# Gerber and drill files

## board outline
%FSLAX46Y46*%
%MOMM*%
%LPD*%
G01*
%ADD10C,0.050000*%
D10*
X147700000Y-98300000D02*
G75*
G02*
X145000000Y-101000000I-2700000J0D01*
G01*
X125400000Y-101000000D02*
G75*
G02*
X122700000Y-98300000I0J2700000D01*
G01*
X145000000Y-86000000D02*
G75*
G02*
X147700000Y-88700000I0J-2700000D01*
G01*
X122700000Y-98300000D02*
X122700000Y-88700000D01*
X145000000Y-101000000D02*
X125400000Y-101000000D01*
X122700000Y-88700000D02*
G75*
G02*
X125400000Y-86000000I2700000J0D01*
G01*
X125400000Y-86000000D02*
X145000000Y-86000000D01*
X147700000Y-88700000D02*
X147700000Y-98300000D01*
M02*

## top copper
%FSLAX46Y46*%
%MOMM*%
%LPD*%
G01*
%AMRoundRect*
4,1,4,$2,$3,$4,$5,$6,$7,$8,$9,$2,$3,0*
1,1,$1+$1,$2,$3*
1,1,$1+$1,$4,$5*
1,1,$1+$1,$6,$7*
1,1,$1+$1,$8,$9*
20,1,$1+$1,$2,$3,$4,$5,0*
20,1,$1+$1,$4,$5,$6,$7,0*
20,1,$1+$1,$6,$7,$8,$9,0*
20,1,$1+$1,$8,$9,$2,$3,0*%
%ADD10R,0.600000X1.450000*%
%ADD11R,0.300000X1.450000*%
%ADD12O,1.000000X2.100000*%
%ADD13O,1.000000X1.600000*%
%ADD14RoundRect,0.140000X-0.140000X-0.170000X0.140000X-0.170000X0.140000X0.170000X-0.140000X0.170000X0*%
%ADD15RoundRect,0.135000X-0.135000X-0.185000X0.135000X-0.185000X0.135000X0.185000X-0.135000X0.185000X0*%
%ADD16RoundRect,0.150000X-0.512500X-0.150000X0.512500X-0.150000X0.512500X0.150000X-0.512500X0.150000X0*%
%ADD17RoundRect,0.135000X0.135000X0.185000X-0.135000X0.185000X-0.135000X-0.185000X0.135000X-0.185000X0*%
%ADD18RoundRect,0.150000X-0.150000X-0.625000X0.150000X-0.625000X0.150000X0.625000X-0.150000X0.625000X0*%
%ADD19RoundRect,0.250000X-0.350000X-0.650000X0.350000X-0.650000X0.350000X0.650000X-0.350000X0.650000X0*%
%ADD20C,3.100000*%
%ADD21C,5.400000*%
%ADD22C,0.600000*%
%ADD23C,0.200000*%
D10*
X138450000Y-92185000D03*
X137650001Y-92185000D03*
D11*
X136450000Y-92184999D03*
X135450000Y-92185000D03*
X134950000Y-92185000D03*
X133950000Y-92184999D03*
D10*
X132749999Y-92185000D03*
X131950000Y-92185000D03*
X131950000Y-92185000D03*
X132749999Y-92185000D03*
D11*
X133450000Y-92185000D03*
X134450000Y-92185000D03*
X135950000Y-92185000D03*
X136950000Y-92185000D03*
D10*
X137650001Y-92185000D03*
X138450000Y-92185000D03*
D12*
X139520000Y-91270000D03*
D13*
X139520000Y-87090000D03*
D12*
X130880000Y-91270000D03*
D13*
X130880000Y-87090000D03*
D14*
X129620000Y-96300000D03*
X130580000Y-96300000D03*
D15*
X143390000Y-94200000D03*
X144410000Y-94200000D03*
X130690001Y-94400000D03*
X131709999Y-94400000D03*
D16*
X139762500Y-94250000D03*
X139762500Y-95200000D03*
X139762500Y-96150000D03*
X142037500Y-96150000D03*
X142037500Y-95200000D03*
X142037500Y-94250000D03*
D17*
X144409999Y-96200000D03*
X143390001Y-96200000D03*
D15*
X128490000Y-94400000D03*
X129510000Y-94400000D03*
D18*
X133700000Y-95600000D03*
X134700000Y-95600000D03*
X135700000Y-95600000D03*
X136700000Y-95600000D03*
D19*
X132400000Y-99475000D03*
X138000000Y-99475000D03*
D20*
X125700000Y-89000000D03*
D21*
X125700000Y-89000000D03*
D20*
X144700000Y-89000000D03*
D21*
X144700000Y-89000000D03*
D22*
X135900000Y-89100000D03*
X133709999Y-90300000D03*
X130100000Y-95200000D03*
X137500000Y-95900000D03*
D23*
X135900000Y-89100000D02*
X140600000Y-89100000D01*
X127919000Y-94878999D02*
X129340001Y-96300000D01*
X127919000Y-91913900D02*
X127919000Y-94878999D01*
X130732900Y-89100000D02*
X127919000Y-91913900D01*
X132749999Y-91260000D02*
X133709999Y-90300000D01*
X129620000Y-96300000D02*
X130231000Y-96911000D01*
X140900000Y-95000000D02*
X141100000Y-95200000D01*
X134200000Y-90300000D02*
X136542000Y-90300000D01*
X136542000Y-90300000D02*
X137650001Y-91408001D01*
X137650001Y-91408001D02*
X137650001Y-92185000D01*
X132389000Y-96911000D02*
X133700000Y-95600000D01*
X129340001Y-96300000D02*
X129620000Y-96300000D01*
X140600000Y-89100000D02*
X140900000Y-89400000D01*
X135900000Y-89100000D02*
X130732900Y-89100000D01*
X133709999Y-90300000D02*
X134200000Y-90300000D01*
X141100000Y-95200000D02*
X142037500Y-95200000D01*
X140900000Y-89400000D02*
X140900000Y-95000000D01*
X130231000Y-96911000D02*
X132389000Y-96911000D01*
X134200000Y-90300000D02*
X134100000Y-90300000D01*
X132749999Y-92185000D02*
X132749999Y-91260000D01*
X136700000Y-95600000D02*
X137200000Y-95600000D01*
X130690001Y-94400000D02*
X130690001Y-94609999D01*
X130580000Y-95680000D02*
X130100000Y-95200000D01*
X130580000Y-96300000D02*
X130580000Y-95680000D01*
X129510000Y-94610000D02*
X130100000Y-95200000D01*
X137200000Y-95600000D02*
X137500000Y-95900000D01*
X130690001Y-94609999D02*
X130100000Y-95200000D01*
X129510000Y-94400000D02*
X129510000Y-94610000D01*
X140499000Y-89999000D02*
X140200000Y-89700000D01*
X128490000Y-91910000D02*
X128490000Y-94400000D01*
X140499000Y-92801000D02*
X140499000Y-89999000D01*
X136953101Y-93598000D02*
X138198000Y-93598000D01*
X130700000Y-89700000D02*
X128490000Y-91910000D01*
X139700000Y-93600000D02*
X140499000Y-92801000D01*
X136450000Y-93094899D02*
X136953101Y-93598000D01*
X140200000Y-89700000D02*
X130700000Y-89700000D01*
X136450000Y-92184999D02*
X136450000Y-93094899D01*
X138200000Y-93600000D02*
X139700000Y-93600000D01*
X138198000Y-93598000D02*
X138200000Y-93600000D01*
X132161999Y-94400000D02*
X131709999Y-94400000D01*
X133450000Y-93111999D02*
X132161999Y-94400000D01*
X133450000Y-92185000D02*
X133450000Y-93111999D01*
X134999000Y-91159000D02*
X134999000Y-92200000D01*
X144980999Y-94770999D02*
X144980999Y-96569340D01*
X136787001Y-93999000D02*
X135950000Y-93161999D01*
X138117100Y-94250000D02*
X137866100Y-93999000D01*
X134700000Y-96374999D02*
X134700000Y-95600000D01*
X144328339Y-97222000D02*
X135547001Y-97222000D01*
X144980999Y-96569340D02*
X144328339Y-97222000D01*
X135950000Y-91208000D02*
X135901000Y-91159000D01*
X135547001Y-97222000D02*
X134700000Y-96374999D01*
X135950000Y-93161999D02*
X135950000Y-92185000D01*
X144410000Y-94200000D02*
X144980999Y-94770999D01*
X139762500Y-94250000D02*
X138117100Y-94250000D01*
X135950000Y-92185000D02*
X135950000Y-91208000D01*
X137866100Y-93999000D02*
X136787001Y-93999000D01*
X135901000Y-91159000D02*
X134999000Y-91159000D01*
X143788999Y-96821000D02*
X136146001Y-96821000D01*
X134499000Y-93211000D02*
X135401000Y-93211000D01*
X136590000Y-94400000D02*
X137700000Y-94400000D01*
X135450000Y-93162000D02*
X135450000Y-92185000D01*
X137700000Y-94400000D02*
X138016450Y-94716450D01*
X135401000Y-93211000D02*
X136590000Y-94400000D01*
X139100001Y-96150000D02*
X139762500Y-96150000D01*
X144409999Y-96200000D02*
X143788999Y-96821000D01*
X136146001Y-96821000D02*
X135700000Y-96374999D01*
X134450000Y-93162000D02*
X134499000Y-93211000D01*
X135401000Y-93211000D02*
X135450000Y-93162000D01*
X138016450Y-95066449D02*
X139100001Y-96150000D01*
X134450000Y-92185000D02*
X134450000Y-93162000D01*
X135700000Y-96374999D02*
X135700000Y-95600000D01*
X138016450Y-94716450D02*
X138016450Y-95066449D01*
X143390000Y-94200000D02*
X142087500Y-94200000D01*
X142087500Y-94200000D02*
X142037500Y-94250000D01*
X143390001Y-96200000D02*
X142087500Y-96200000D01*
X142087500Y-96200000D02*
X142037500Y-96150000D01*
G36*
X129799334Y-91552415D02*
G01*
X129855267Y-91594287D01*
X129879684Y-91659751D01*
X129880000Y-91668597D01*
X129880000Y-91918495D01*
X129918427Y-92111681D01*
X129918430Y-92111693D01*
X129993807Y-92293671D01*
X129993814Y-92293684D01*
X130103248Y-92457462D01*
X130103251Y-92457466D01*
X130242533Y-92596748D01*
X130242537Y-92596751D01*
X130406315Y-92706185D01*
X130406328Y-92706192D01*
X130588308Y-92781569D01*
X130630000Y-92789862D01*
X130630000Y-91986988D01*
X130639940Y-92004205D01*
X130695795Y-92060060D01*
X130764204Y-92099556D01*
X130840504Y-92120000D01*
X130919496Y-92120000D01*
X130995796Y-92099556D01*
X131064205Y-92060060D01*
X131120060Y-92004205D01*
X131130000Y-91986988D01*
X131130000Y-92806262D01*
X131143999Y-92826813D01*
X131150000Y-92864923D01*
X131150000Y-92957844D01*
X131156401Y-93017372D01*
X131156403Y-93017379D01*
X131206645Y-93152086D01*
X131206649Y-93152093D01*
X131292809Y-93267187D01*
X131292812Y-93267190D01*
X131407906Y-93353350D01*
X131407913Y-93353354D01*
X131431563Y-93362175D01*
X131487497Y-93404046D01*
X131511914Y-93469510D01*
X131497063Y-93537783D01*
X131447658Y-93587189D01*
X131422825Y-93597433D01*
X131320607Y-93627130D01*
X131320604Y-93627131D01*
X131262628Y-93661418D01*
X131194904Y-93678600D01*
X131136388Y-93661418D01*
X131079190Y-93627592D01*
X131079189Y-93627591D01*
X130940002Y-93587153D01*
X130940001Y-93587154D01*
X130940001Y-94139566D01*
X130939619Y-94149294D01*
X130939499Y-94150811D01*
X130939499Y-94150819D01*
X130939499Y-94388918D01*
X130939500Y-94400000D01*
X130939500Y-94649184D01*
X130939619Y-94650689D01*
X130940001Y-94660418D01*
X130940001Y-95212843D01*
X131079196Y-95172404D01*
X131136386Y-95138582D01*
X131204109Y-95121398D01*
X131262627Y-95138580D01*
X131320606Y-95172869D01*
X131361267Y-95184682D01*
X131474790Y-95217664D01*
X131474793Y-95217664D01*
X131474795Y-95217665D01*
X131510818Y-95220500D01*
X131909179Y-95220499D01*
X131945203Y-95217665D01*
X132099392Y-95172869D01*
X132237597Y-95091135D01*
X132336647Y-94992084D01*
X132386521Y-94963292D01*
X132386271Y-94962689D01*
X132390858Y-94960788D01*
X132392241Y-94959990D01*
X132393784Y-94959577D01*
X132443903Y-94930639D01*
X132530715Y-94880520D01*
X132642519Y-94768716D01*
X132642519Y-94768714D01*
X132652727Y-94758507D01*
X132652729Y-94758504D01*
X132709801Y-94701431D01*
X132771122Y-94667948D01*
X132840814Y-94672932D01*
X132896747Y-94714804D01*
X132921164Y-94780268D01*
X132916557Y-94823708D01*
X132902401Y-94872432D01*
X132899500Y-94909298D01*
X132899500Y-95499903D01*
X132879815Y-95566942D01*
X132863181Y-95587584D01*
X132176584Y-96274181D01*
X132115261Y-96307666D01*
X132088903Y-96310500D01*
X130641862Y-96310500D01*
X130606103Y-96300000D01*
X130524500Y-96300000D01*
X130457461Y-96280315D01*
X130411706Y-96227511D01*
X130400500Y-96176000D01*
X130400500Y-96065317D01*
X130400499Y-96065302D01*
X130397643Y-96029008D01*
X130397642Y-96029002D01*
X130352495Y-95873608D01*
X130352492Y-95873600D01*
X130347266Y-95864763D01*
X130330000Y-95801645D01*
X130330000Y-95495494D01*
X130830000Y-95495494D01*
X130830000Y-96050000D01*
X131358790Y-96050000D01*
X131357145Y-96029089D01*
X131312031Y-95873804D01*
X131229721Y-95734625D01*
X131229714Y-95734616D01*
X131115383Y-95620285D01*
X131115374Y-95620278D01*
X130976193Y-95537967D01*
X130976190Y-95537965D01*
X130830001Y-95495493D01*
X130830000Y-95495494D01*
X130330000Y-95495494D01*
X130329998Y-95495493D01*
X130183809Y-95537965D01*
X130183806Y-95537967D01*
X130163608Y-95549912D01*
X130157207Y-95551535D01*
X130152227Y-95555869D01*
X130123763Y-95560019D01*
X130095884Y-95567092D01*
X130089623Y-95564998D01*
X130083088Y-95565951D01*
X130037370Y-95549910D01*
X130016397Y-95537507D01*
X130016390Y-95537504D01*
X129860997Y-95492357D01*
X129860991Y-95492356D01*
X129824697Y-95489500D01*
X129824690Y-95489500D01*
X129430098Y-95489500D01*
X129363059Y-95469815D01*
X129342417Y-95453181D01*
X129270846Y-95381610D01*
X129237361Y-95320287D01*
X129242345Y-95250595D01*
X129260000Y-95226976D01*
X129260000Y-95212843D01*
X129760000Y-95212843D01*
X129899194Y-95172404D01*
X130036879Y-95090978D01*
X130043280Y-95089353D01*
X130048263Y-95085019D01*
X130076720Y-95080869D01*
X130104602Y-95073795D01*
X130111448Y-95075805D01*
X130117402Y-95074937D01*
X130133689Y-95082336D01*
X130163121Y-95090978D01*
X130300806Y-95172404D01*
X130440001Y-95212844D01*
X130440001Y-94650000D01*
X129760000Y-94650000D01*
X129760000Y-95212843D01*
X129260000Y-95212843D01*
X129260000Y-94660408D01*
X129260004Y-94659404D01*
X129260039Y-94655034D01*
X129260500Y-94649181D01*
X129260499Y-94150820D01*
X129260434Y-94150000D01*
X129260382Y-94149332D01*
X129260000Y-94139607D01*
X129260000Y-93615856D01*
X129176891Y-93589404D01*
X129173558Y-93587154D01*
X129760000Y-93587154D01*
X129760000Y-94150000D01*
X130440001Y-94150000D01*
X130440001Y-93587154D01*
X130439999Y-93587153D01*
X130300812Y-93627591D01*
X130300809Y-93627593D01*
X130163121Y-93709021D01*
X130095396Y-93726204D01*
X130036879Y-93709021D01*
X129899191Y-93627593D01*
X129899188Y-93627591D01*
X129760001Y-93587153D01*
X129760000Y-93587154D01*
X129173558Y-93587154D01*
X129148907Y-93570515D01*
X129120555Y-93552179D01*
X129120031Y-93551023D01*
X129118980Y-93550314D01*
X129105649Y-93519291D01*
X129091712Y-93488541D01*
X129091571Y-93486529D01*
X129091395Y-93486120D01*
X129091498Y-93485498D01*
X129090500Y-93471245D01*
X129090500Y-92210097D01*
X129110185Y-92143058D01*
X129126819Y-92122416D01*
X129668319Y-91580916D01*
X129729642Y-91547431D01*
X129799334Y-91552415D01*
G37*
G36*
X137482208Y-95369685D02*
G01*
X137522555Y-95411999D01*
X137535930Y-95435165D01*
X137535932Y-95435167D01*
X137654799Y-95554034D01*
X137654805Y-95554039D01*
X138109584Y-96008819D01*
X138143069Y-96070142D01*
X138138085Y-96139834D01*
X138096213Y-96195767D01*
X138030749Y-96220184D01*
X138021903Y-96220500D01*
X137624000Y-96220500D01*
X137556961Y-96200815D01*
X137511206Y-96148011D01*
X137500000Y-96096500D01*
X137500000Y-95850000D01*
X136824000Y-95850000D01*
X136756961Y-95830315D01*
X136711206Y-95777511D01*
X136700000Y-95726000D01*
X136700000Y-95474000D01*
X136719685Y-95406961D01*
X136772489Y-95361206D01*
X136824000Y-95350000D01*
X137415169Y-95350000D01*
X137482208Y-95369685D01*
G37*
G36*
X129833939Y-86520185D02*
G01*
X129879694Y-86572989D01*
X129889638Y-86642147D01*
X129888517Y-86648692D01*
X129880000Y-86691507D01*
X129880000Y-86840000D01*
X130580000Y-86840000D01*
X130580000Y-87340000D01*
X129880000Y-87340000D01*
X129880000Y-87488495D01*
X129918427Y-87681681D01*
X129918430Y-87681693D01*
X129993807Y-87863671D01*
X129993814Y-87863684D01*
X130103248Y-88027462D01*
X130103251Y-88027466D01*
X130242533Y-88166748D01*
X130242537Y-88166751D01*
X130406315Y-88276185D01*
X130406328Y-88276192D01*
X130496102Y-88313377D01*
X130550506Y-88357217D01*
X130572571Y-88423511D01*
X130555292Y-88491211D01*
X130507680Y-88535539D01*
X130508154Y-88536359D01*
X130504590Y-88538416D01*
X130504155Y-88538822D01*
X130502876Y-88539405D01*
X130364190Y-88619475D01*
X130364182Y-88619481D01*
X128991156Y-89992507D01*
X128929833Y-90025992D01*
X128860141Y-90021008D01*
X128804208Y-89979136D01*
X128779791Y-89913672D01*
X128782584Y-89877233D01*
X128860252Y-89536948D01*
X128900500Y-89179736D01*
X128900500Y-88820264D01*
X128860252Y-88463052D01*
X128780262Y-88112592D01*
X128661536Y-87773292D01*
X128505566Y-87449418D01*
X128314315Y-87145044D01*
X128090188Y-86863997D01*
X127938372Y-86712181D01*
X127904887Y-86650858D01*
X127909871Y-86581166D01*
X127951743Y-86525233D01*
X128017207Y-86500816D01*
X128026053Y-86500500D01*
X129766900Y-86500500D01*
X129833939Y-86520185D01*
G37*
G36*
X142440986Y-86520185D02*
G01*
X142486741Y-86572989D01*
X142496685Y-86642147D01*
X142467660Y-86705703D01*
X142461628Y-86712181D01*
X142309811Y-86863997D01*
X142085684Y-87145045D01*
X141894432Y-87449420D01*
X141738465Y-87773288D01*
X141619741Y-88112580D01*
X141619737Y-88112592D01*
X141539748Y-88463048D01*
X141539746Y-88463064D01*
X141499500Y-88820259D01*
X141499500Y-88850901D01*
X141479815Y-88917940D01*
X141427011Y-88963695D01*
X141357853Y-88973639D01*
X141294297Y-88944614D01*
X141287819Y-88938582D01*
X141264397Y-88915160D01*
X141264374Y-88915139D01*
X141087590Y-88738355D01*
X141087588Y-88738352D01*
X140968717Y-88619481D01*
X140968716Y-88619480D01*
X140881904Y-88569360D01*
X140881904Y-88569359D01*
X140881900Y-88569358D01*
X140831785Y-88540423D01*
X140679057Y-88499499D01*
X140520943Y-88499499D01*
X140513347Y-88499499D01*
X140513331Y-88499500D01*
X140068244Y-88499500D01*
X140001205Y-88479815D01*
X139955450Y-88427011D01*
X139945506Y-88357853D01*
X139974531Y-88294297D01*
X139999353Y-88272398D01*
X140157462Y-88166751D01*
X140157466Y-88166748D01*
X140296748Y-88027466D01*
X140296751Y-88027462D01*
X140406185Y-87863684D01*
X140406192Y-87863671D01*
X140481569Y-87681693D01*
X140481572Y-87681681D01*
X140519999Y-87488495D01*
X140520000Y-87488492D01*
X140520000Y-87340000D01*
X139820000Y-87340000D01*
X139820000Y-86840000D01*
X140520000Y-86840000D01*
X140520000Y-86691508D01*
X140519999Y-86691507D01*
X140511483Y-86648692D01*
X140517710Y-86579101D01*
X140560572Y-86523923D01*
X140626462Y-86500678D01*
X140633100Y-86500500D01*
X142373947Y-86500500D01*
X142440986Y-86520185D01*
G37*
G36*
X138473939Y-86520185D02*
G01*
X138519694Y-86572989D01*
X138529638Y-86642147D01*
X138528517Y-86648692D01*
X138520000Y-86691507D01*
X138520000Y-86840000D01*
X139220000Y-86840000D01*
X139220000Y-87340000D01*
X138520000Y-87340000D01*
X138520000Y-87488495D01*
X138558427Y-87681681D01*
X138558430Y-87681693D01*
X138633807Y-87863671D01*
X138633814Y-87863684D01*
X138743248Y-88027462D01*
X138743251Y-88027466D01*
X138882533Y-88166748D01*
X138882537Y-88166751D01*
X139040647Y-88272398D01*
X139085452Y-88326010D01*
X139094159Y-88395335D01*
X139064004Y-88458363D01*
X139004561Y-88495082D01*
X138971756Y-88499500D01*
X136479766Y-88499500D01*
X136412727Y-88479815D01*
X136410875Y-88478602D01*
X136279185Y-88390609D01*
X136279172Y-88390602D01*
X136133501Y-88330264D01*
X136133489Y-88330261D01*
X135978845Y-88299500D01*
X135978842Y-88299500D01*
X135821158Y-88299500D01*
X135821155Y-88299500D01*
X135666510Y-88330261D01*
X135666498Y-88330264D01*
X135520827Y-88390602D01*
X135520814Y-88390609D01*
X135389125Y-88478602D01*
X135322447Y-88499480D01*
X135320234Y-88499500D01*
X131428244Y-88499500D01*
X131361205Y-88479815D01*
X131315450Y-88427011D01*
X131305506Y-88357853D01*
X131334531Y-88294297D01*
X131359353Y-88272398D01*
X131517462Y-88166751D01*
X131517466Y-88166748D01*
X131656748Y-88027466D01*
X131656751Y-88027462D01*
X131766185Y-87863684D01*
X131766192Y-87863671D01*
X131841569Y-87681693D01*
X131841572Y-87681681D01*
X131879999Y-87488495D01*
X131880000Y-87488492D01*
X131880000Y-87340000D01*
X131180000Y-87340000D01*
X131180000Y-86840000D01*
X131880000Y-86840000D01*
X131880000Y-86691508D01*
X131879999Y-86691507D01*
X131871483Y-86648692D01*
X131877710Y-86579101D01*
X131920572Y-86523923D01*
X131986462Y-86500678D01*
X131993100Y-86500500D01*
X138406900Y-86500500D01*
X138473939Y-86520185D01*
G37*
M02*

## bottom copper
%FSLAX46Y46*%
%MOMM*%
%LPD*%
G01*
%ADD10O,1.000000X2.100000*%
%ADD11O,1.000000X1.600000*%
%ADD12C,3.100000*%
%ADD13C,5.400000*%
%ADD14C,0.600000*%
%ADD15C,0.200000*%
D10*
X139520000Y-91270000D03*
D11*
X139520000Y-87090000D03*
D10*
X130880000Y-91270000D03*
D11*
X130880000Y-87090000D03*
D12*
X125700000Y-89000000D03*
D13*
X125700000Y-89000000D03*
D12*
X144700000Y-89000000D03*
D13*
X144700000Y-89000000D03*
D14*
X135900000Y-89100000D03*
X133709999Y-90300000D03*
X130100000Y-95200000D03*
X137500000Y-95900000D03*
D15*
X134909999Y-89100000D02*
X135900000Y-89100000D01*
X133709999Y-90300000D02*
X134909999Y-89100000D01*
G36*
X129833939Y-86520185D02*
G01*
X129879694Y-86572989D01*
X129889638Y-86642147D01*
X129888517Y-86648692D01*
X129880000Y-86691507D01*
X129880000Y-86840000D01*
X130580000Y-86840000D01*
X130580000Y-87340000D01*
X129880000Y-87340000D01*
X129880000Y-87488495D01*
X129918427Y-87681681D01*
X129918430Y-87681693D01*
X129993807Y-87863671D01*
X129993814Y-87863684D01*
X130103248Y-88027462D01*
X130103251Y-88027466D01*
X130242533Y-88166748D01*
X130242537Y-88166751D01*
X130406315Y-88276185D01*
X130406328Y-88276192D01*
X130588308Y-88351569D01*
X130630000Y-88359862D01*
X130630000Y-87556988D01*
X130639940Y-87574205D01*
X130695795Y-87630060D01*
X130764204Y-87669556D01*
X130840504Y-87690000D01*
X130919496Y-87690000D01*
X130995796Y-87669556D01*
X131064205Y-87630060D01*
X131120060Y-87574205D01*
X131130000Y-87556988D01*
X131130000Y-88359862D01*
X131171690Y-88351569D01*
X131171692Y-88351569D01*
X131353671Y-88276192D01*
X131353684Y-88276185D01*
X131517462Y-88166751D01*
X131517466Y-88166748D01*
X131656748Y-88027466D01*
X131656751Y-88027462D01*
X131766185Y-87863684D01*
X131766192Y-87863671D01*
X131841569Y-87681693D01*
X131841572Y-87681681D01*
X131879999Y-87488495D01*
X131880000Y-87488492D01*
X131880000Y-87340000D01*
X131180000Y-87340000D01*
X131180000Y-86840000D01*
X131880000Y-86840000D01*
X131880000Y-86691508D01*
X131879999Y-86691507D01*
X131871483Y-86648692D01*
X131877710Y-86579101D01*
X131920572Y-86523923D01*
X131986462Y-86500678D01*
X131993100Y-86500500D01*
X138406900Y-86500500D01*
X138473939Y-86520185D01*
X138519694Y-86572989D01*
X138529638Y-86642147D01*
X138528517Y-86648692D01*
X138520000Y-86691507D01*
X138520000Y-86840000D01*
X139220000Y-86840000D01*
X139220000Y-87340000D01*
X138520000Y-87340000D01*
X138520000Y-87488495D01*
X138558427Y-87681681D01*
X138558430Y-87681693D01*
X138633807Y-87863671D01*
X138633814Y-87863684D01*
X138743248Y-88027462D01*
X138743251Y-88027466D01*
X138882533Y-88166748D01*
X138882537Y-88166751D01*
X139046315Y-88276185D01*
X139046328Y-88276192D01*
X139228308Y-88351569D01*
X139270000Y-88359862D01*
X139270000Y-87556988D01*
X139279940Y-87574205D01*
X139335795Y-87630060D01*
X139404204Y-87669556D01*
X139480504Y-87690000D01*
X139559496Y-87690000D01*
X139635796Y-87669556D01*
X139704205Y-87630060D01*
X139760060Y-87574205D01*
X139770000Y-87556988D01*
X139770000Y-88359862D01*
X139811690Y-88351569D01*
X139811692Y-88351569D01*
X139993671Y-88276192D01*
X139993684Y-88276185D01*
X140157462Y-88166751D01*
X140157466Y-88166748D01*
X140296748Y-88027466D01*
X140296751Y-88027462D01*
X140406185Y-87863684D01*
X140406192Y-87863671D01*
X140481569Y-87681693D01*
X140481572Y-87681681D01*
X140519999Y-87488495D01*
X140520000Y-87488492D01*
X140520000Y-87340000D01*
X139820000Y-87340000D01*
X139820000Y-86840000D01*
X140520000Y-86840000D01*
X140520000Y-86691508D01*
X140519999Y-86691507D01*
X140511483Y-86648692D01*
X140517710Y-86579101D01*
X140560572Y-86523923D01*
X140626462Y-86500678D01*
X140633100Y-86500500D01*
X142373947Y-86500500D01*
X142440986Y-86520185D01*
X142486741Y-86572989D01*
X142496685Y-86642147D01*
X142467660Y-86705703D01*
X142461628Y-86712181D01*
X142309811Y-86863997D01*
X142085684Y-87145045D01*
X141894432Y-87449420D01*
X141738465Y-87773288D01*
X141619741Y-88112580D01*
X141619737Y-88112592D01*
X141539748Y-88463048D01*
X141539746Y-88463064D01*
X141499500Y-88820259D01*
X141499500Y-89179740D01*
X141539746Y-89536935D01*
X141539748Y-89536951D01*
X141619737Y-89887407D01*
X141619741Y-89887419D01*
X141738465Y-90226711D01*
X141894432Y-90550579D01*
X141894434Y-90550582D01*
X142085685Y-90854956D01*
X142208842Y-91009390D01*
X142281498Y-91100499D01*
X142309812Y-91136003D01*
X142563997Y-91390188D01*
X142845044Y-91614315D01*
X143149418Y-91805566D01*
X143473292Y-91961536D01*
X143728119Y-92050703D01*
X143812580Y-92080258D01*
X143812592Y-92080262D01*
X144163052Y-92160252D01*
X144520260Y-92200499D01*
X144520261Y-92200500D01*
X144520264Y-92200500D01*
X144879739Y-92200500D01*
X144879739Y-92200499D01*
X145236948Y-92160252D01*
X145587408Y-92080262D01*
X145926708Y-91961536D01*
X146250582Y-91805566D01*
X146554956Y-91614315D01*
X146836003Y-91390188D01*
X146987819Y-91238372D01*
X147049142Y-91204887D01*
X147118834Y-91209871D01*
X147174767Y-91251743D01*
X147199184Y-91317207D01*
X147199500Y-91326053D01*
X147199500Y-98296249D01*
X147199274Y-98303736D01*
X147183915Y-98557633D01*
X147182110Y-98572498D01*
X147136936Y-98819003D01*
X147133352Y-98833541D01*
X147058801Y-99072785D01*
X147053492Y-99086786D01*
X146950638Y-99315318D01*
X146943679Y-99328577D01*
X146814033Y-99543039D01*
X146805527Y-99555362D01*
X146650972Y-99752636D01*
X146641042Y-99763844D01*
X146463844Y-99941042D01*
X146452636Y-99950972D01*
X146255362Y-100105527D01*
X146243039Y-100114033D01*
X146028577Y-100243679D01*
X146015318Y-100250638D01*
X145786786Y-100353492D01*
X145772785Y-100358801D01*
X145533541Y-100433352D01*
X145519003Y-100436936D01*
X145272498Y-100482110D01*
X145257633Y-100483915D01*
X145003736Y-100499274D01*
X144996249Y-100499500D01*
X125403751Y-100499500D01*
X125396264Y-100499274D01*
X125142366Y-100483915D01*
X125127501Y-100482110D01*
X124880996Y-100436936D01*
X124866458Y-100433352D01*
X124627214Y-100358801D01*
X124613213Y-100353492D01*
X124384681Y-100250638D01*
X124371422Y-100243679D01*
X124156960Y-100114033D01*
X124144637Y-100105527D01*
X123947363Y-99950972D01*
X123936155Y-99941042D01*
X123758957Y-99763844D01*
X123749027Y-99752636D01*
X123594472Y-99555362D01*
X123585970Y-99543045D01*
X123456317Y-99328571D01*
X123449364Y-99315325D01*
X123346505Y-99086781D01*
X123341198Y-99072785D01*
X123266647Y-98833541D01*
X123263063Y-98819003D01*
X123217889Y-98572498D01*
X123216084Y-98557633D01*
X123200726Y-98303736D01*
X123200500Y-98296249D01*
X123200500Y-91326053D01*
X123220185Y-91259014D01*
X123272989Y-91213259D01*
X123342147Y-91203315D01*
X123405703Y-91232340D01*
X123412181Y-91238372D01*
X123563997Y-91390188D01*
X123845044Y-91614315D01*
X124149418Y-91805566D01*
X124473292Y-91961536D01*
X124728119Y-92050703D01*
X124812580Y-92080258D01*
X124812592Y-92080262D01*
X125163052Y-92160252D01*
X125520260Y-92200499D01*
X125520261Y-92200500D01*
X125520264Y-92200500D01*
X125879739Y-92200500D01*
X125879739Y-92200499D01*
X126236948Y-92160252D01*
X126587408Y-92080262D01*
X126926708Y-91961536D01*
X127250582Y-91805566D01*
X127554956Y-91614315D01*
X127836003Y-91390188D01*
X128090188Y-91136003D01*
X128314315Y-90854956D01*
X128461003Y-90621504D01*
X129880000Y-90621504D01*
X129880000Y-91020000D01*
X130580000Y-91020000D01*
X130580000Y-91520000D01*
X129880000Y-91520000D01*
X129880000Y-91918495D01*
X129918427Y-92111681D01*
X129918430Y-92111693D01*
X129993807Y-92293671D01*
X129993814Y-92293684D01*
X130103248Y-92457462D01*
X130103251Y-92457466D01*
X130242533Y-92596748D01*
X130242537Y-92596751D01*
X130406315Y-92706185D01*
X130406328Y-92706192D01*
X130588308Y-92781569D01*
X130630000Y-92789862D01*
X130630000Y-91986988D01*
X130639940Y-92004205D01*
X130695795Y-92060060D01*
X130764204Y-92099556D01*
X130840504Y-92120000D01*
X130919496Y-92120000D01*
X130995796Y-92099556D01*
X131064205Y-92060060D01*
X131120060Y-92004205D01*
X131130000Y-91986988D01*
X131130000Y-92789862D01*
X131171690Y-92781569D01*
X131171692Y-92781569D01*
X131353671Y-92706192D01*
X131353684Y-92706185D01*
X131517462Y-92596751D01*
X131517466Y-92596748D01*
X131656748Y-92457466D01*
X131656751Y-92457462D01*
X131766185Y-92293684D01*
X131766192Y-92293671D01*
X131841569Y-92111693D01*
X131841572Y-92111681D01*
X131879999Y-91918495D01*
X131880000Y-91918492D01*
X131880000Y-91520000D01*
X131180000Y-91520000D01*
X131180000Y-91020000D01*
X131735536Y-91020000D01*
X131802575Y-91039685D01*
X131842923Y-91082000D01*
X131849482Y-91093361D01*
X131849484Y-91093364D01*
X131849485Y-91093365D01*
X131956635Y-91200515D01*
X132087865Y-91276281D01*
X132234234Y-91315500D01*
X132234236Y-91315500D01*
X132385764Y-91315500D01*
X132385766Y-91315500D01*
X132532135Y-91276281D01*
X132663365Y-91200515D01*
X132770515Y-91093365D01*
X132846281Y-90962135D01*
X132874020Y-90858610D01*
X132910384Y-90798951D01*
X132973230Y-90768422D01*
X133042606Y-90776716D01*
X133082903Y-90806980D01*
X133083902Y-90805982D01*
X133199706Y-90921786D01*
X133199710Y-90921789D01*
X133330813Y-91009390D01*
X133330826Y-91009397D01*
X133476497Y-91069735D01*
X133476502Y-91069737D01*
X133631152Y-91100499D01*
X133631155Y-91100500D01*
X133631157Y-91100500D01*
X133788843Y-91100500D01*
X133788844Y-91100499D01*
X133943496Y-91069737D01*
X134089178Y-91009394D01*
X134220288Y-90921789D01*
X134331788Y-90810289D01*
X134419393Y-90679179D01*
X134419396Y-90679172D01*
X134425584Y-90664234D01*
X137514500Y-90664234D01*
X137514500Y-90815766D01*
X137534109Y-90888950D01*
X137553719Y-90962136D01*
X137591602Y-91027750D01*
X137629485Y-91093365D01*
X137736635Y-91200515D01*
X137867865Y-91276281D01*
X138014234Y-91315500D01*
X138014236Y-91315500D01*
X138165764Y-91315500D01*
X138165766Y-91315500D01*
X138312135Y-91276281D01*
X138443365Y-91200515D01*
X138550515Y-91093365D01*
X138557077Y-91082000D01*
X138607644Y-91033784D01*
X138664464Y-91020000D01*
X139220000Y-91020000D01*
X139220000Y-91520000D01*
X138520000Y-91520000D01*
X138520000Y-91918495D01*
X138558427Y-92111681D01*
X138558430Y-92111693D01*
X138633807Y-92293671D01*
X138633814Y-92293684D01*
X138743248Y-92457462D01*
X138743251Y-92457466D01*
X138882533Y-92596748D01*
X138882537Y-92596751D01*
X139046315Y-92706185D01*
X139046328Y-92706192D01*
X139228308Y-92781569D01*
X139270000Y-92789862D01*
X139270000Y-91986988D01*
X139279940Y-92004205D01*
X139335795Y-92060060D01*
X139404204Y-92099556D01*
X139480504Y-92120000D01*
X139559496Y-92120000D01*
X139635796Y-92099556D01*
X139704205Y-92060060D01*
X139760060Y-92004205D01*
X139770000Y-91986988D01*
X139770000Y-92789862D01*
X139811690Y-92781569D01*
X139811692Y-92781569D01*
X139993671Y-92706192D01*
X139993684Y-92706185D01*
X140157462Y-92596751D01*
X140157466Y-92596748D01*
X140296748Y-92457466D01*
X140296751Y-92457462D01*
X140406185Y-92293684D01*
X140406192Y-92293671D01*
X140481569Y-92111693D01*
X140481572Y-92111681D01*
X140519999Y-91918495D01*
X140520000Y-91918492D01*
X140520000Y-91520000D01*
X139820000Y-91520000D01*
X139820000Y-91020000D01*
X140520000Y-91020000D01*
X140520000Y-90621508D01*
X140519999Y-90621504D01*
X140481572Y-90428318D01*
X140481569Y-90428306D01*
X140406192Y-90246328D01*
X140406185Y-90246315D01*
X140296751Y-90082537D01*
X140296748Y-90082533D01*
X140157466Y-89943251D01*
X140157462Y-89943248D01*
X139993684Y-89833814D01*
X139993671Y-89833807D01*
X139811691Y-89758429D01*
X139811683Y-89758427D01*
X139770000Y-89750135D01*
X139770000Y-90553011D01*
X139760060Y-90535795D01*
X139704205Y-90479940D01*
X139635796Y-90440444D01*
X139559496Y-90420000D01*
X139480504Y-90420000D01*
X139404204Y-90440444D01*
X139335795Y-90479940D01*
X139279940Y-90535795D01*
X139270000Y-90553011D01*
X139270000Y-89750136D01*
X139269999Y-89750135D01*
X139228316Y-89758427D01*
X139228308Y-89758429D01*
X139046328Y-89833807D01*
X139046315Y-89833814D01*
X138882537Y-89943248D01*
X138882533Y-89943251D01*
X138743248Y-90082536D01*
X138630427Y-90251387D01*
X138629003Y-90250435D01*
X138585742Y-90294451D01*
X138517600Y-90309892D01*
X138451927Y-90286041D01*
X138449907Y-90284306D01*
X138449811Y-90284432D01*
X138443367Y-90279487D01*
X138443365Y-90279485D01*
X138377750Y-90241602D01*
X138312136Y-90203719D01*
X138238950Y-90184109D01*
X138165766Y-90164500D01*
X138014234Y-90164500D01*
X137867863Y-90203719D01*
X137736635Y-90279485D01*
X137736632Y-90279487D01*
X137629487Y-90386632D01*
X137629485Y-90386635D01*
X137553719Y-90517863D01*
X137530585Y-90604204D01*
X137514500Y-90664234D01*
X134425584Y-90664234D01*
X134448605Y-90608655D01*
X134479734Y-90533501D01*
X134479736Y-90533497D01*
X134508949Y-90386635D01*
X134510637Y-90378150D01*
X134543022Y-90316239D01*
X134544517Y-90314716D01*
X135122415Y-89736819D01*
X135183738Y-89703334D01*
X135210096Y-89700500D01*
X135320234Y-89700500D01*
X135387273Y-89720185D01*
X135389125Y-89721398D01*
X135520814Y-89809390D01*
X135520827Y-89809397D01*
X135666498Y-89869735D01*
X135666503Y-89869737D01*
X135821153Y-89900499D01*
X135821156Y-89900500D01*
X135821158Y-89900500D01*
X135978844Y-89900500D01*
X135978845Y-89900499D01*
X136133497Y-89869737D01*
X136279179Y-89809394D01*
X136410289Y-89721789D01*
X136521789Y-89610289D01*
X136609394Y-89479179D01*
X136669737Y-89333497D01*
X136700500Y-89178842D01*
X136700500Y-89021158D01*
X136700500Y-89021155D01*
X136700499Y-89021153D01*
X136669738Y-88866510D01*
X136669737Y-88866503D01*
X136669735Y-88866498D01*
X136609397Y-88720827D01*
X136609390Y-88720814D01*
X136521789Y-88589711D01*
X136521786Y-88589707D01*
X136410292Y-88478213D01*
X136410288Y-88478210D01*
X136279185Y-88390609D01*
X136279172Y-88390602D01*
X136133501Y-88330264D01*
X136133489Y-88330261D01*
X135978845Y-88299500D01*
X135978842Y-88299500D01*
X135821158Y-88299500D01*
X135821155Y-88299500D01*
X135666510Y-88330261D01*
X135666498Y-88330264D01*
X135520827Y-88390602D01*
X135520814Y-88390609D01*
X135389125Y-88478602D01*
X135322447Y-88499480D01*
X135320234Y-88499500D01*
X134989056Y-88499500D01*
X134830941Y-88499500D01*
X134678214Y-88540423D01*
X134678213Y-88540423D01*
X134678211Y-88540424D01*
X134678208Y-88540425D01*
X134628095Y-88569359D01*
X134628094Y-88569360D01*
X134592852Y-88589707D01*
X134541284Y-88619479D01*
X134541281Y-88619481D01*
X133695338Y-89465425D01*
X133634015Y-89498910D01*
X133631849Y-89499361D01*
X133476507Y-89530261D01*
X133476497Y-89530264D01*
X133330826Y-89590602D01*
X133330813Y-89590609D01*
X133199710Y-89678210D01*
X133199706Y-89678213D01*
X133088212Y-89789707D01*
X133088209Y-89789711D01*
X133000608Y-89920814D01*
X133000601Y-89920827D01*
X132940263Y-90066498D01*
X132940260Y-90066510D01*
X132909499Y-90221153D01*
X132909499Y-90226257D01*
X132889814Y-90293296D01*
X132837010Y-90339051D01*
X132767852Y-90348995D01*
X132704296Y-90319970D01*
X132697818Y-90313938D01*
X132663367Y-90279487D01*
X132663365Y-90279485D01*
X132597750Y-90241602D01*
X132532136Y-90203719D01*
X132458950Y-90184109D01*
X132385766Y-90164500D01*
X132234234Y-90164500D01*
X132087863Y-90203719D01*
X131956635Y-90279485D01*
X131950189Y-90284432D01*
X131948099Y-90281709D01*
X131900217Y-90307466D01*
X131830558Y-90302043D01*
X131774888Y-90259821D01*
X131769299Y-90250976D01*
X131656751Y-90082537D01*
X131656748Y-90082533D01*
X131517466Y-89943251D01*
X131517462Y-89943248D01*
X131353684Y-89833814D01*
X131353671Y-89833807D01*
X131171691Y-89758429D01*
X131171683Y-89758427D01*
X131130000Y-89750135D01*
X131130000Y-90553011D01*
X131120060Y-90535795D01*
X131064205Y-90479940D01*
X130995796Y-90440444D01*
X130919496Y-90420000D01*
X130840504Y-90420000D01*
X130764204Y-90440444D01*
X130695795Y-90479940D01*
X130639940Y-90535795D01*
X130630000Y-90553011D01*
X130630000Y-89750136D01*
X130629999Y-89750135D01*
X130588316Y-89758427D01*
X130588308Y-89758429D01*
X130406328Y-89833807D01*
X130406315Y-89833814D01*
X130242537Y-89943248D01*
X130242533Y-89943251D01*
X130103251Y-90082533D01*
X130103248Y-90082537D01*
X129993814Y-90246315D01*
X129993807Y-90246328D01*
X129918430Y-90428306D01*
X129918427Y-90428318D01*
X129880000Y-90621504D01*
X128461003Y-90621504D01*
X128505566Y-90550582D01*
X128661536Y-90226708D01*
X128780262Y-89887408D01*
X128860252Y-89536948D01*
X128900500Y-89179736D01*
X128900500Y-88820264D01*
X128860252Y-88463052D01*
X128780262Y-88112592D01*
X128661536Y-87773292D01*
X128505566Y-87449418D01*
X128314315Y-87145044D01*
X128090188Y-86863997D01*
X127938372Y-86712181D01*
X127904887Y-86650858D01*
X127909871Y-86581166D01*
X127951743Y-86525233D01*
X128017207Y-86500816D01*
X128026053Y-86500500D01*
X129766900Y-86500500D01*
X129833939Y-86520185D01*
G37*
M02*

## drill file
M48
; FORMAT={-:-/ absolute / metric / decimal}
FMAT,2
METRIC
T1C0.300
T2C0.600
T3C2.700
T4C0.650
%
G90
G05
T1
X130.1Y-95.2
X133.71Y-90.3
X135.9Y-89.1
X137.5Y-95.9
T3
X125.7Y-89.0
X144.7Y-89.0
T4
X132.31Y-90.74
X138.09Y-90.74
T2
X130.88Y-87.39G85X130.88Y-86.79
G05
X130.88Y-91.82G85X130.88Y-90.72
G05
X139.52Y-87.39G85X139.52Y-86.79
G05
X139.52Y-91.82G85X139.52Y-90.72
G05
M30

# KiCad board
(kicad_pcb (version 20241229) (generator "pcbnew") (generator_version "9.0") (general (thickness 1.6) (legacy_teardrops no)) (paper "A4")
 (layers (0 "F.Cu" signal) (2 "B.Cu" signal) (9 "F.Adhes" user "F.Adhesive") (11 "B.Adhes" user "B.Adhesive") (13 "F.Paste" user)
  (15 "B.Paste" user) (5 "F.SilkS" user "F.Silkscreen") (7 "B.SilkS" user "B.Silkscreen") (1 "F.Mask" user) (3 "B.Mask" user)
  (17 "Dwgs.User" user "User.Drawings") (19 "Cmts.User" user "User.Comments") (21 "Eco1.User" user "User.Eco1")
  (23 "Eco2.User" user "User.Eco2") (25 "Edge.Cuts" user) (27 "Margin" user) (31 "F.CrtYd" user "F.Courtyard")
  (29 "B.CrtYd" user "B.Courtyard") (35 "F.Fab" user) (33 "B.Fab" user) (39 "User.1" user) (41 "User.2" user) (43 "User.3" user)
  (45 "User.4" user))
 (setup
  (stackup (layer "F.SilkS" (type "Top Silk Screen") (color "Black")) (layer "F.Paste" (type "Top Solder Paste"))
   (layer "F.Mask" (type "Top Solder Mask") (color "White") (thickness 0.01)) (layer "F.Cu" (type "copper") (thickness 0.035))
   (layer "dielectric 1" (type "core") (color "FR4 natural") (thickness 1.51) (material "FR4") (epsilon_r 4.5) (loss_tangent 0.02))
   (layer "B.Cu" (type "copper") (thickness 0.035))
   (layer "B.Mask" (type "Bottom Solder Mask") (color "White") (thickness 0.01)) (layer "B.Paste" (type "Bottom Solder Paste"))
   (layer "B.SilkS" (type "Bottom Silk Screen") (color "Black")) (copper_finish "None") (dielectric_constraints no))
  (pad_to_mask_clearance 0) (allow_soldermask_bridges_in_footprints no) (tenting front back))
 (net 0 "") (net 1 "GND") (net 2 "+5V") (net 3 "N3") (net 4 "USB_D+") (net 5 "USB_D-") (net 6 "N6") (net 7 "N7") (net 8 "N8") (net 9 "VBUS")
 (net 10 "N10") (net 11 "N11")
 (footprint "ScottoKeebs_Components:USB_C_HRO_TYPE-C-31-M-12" (layer "F.Cu") (at 135.2 88.14 180)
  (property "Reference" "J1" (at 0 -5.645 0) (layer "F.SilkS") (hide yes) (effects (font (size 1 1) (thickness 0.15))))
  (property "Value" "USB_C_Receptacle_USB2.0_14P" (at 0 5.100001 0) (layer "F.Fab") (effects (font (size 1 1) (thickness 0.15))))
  (pad "" np_thru_hole circle (at -2.89 -2.6 180) (size 0.65 0.65) (drill 0.65) (layers "*.Cu" "*.Mask"))
  (pad "" np_thru_hole circle (at 2.89 -2.6 180) (size 0.65 0.65) (drill 0.65) (layers "*.Cu" "*.Mask"))
  (pad "A1" smd rect (at -3.25 -4.045 180) (size 0.6 1.45) (layers "F.Cu" "F.Mask" "F.Paste") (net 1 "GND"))
  (pad "A4" smd rect (at -2.450001 -4.045 180) (size 0.6 1.45) (layers "F.Cu" "F.Mask" "F.Paste") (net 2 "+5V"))
  (pad "A5" smd rect (at -1.25 -4.044999 180) (size 0.3 1.45) (layers "F.Cu" "F.Mask" "F.Paste") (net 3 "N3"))
  (pad "A6" smd rect (at -0.25 -4.045 180) (size 0.3 1.45) (layers "F.Cu" "F.Mask" "F.Paste") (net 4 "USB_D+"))
  (pad "A7" smd rect (at 0.25 -4.045 180) (size 0.3 1.45) (layers "F.Cu" "F.Mask" "F.Paste") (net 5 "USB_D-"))
  (pad "A8" smd rect (at 1.25 -4.044999 180) (size 0.3 1.45) (layers "F.Cu" "F.Mask" "F.Paste"))
  (pad "A9" smd rect (at 2.450001 -4.045 180) (size 0.6 1.45) (layers "F.Cu" "F.Mask" "F.Paste") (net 2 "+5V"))
  (pad "A12" smd rect (at 3.25 -4.045 180) (size 0.6 1.45) (layers "F.Cu" "F.Mask" "F.Paste") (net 1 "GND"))
  (pad "B1" smd rect (at 3.25 -4.045 180) (size 0.6 1.45) (layers "F.Cu" "F.Mask" "F.Paste") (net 1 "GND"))
  (pad "B4" smd rect (at 2.450001 -4.045 180) (size 0.6 1.45) (layers "F.Cu" "F.Mask" "F.Paste") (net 2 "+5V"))
  (pad "B5" smd rect (at 1.75 -4.045 180) (size 0.3 1.45) (layers "F.Cu" "F.Mask" "F.Paste") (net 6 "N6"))
  (pad "B6" smd rect (at 0.75 -4.045 180) (size 0.3 1.45) (layers "F.Cu" "F.Mask" "F.Paste") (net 4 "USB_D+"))
  (pad "B7" smd rect (at -0.75 -4.045 180) (size 0.3 1.45) (layers "F.Cu" "F.Mask" "F.Paste") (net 5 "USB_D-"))
  (pad "B8" smd rect (at -1.75 -4.045 180) (size 0.3 1.45) (layers "F.Cu" "F.Mask" "F.Paste"))
  (pad "B9" smd rect (at -2.450001 -4.045 180) (size 0.6 1.45) (layers "F.Cu" "F.Mask" "F.Paste") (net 2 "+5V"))
  (pad "B12" smd rect (at -3.25 -4.045 180) (size 0.6 1.45) (layers "F.Cu" "F.Mask" "F.Paste") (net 1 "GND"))
  (pad "S1" thru_hole oval (at -4.32 -3.13 180) (size 1 2.1) (drill oval 0.6 1.7) (layers "*.Cu" "*.Mask") (remove_unused_layers no)
   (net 1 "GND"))
  (pad "S1" thru_hole oval (at -4.32 1.05 180) (size 1 1.6) (drill oval 0.6 1.2) (layers "*.Cu" "*.Mask") (remove_unused_layers no)
   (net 1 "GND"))
  (pad "S1" thru_hole oval (at 4.32 -3.13 180) (size 1 2.1) (drill oval 0.6 1.7) (layers "*.Cu" "*.Mask") (remove_unused_layers no)
   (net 1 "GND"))
  (pad "S1" thru_hole oval (at 4.32 1.05 180) (size 1 1.6) (drill oval 0.6 1.2) (layers "*.Cu" "*.Mask") (remove_unused_layers no)
   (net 1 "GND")))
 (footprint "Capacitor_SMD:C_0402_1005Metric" (layer "F.Cu") (at 130.1 96.3)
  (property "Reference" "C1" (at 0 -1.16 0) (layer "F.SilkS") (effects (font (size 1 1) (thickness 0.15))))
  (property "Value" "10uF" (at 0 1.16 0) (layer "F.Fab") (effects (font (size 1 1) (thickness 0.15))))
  (pad "1" smd roundrect (at -0.48 0) (size 0.56 0.62) (layers "F.Cu" "F.Mask" "F.Paste") (roundrect_rratio 0.25) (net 2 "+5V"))
  (pad "2" smd roundrect (at 0.48 0) (size 0.56 0.62) (layers "F.Cu" "F.Mask" "F.Paste") (roundrect_rratio 0.25) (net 1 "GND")))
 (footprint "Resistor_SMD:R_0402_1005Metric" (layer "F.Cu") (at 143.9 94.2)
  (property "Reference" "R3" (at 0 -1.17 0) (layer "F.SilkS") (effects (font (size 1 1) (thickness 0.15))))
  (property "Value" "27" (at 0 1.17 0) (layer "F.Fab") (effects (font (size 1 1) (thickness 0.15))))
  (pad "1" smd roundrect (at -0.51 0) (size 0.54 0.64) (layers "F.Cu" "F.Mask" "F.Paste") (roundrect_rratio 0.25) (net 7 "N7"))
  (pad "2" smd roundrect (at 0.51 0) (size 0.54 0.64) (layers "F.Cu" "F.Mask" "F.Paste") (roundrect_rratio 0.25) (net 4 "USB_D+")))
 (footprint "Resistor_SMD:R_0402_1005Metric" (layer "F.Cu") (at 131.2 94.4)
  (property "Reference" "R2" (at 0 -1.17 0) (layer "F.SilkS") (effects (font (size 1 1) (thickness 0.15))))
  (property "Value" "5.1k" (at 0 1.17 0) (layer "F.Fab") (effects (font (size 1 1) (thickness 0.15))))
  (pad "1" smd roundrect (at -0.509999 0) (size 0.54 0.64) (layers "F.Cu" "F.Mask" "F.Paste") (roundrect_rratio 0.25) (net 1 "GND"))
  (pad "2" smd roundrect (at 0.509999 0) (size 0.54 0.64) (layers "F.Cu" "F.Mask" "F.Paste") (roundrect_rratio 0.25) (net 6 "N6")))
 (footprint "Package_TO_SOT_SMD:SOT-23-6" (layer "F.Cu") (at 140.9 95.2)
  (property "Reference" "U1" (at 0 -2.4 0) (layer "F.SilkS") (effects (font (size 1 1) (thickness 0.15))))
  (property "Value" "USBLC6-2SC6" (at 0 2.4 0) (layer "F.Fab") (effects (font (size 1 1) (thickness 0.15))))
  (pad "1" smd roundrect (at -1.1375 -0.95) (size 1.325 0.6) (layers "F.Cu" "F.Mask" "F.Paste") (roundrect_rratio 0.25) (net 4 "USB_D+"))
  (pad "2" smd roundrect (at -1.1375 0) (size 1.325 0.6) (layers "F.Cu" "F.Mask" "F.Paste") (roundrect_rratio 0.25) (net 1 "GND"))
  (pad "3" smd roundrect (at -1.1375 0.95) (size 1.325 0.6) (layers "F.Cu" "F.Mask" "F.Paste") (roundrect_rratio 0.25) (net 5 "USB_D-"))
  (pad "4" smd roundrect (at 1.1375 0.95) (size 1.325 0.6) (layers "F.Cu" "F.Mask" "F.Paste") (roundrect_rratio 0.25) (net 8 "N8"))
  (pad "5" smd roundrect (at 1.1375 0) (size 1.325 0.6) (layers "F.Cu" "F.Mask" "F.Paste") (roundrect_rratio 0.25) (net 2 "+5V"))
  (pad "6" smd roundrect (at 1.1375 -0.95) (size 1.325 0.6) (layers "F.Cu" "F.Mask" "F.Paste") (roundrect_rratio 0.25) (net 7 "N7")))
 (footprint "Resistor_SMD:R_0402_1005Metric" (layer "F.Cu") (at 143.9 96.2 180)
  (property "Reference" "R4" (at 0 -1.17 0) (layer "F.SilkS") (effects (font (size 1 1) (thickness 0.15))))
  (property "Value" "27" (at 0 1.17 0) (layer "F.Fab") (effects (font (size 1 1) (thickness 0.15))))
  (pad "1" smd roundrect (at -0.509999 0 180) (size 0.54 0.64) (layers "F.Cu" "F.Mask" "F.Paste") (roundrect_rratio 0.25) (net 5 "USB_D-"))
  (pad "2" smd roundrect (at 0.509999 0 180) (size 0.54 0.64) (layers "F.Cu" "F.Mask" "F.Paste") (roundrect_rratio 0.25) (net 8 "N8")))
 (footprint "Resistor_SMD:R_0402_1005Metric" (layer "F.Cu") (at 129 94.4)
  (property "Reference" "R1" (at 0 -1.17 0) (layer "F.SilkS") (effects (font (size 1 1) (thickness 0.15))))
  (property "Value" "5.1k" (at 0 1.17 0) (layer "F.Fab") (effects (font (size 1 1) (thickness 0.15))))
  (pad "1" smd roundrect (at -0.51 0) (size 0.54 0.64) (layers "F.Cu" "F.Mask" "F.Paste") (roundrect_rratio 0.25) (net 3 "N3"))
  (pad "2" smd roundrect (at 0.51 0) (size 0.54 0.64) (layers "F.Cu" "F.Mask" "F.Paste") (roundrect_rratio 0.25) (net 1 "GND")))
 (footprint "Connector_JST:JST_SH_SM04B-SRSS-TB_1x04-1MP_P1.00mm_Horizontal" (layer "F.Cu") (at 135.2 97.6)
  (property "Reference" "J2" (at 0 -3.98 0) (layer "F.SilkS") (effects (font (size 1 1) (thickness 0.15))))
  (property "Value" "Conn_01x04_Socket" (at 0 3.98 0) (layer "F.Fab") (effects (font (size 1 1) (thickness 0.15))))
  (pad "1" smd roundrect (at -1.5 -2) (size 0.6 1.55) (layers "F.Cu" "F.Mask" "F.Paste") (roundrect_rratio 0.25) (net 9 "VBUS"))
  (pad "2" smd roundrect (at -0.5 -2) (size 0.6 1.55) (layers "F.Cu" "F.Mask" "F.Paste") (roundrect_rratio 0.25) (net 5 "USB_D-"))
  (pad "3" smd roundrect (at 0.5 -2) (size 0.6 1.55) (layers "F.Cu" "F.Mask" "F.Paste") (roundrect_rratio 0.25) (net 4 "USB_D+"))
  (pad "4" smd roundrect (at 1.5 -2) (size 0.6 1.55) (layers "F.Cu" "F.Mask" "F.Paste") (roundrect_rratio 0.25) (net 1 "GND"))
  (pad "MP" smd roundrect (at -2.8 1.875) (size 1.2 1.8) (layers "F.Cu" "F.Mask" "F.Paste") (roundrect_rratio 0.208333))
  (pad "MP" smd roundrect (at 2.8 1.875) (size 1.2 1.8) (layers "F.Cu" "F.Mask" "F.Paste") (roundrect_rratio 0.208333)))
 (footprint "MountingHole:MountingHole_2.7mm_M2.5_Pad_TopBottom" (layer "B.Cu") (at 125.7 89 180)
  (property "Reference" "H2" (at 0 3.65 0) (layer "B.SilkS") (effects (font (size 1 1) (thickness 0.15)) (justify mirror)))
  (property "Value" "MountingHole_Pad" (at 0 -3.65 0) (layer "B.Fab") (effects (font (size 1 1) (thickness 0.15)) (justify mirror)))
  (pad "1" thru_hole circle (at 0 0 180) (size 3.1 3.1) (drill 2.7) (layers "*.Cu" "*.Mask") (remove_unused_layers no) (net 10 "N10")
   (zone_connect 2))
  (pad "1" connect circle (at 0 0 180) (size 5.4 5.4) (layers "F.Cu" "F.Mask") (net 10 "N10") (zone_connect 2))
  (pad "1" connect circle (at 0 0 180) (size 5.4 5.4) (layers "B.Cu" "B.Mask") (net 10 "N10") (zone_connect 2)))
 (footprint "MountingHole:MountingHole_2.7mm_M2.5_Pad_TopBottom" (layer "B.Cu") (at 144.7 89 180)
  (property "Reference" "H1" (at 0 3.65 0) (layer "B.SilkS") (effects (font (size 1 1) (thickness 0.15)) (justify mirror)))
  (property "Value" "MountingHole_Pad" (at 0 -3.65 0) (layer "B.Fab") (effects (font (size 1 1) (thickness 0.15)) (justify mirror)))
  (pad "1" thru_hole circle (at 0 0 180) (size 3.1 3.1) (drill 2.7) (layers "*.Cu" "*.Mask") (remove_unused_layers no) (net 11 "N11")
   (zone_connect 2))
  (pad "1" connect circle (at 0 0 180) (size 5.4 5.4) (layers "F.Cu" "F.Mask") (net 11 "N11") (zone_connect 2))
  (pad "1" connect circle (at 0 0 180) (size 5.4 5.4) (layers "B.Cu" "B.Mask") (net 11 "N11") (zone_connect 2)))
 (gr_arc (start 147.7 98.3) (mid 146.909188 100.209188) (end 145 101) (stroke (width 0.05) (type default)) (layer "Edge.Cuts"))
 (gr_arc (start 125.4 101) (mid 123.490812 100.209188) (end 122.7 98.3) (stroke (width 0.05) (type default)) (layer "Edge.Cuts"))
 (gr_arc (start 145 86) (mid 146.909188 86.790812) (end 147.7 88.7) (stroke (width 0.05) (type default)) (layer "Edge.Cuts"))
 (gr_line (start 122.7 98.3) (end 122.7 88.7) (stroke (width 0.05) (type default)) (layer "Edge.Cuts"))
 (gr_line (start 145 101) (end 125.4 101) (stroke (width 0.05) (type default)) (layer "Edge.Cuts"))
 (gr_arc (start 122.7 88.7) (mid 123.490812 86.790812) (end 125.4 86) (stroke (width 0.05) (type default)) (layer "Edge.Cuts"))
 (gr_line (start 125.4 86) (end 145 86) (stroke (width 0.05) (type default)) (layer "Edge.Cuts"))
 (gr_line (start 147.7 88.7) (end 147.7 98.3) (stroke (width 0.05) (type default)) (layer "Edge.Cuts"))
 (segment (start 135.9 89.1) (end 140.6 89.1) (width 0.2) (layer "F.Cu") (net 2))
 (segment (start 127.919 94.878999) (end 129.340001 96.3) (width 0.2) (layer "F.Cu") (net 2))
 (segment (start 127.919 91.9139) (end 127.919 94.878999) (width 0.2) (layer "F.Cu") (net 2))
 (segment (start 130.7329 89.1) (end 127.919 91.9139) (width 0.2) (layer "F.Cu") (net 2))
 (segment (start 132.749999 91.26) (end 133.709999 90.3) (width 0.2) (layer "F.Cu") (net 2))
 (segment (start 129.62 96.3) (end 130.231 96.911) (width 0.2) (layer "F.Cu") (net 2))
 (segment (start 140.9 95) (end 141.1 95.2) (width 0.2) (layer "F.Cu") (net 2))
 (segment (start 134.2 90.3) (end 136.542 90.3) (width 0.2) (layer "F.Cu") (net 2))
 (segment (start 136.542 90.3) (end 137.650001 91.408001) (width 0.2) (layer "F.Cu") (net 2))
 (segment (start 137.650001 91.408001) (end 137.650001 92.185) (width 0.2) (layer "F.Cu") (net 2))
 (segment (start 132.389 96.911) (end 133.7 95.6) (width 0.2) (layer "F.Cu") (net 2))
 (segment (start 129.340001 96.3) (end 129.62 96.3) (width 0.2) (layer "F.Cu") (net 2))
 (segment (start 140.6 89.1) (end 140.9 89.4) (width 0.2) (layer "F.Cu") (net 2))
 (segment (start 135.9 89.1) (end 130.7329 89.1) (width 0.2) (layer "F.Cu") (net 2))
 (segment (start 133.709999 90.3) (end 134.2 90.3) (width 0.2) (layer "F.Cu") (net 2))
 (segment (start 141.1 95.2) (end 142.0375 95.2) (width 0.2) (layer "F.Cu") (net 2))
 (segment (start 140.9 89.4) (end 140.9 95) (width 0.2) (layer "F.Cu") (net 2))
 (segment (start 130.231 96.911) (end 132.389 96.911) (width 0.2) (layer "F.Cu") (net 2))
 (segment (start 134.2 90.3) (end 134.1 90.3) (width 0.2) (layer "F.Cu") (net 2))
 (segment (start 132.749999 92.185) (end 132.749999 91.26) (width 0.2) (layer "F.Cu") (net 2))
 (via (at 135.9 89.1) (size 0.6) (drill 0.3) (layers "F.Cu" "B.Cu") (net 2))
 (via (at 133.709999 90.3) (size 0.6) (drill 0.3) (layers "F.Cu" "B.Cu") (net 2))
 (segment (start 134.909999 89.1) (end 135.9 89.1) (width 0.2) (layer "B.Cu") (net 2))
 (segment (start 133.709999 90.3) (end 134.909999 89.1) (width 0.2) (layer "B.Cu") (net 2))
 (segment (start 136.7 95.6) (end 137.2 95.6) (width 0.2) (layer "F.Cu") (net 1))
 (segment (start 130.690001 94.4) (end 130.690001 94.609999) (width 0.2) (layer "F.Cu") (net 1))
 (segment (start 130.58 95.68) (end 130.1 95.2) (width 0.2) (layer "F.Cu") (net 1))
 (segment (start 130.58 96.3) (end 130.58 95.68) (width 0.2) (layer "F.Cu") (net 1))
 (segment (start 129.51 94.61) (end 130.1 95.2) (width 0.2) (layer "F.Cu") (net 1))
 (segment (start 137.2 95.6) (end 137.5 95.9) (width 0.2) (layer "F.Cu") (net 1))
 (segment (start 130.690001 94.609999) (end 130.1 95.2) (width 0.2) (layer "F.Cu") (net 1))
 (segment (start 129.51 94.4) (end 129.51 94.61) (width 0.2) (layer "F.Cu") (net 1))
 (via (at 130.1 95.2) (size 0.6) (drill 0.3) (layers "F.Cu" "B.Cu") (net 1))
 (via (at 137.5 95.9) (size 0.6) (drill 0.3) (layers "F.Cu" "B.Cu") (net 1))
 (segment (start 140.499 89.999) (end 140.2 89.7) (width 0.2) (layer "F.Cu") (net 3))
 (segment (start 128.49 91.91) (end 128.49 94.4) (width 0.2) (layer "F.Cu") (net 3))
 (segment (start 140.499 92.801) (end 140.499 89.999) (width 0.2) (layer "F.Cu") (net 3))
 (segment (start 136.953101 93.598) (end 138.198 93.598) (width 0.2) (layer "F.Cu") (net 3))
 (segment (start 130.7 89.7) (end 128.49 91.91) (width 0.2) (layer "F.Cu") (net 3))
 (segment (start 139.7 93.6) (end 140.499 92.801) (width 0.2) (layer "F.Cu") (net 3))
 (segment (start 136.45 93.094899) (end 136.953101 93.598) (width 0.2) (layer "F.Cu") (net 3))
 (segment (start 140.2 89.7) (end 130.7 89.7) (width 0.2) (layer "F.Cu") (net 3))
 (segment (start 136.45 92.184999) (end 136.45 93.094899) (width 0.2) (layer "F.Cu") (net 3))
 (segment (start 138.2 93.6) (end 139.7 93.6) (width 0.2) (layer "F.Cu") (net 3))
 (segment (start 138.198 93.598) (end 138.2 93.6) (width 0.2) (layer "F.Cu") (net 3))
 (segment (start 132.161999 94.4) (end 131.709999 94.4) (width 0.2) (layer "F.Cu") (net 6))
 (segment (start 133.45 93.111999) (end 132.161999 94.4) (width 0.2) (layer "F.Cu") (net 6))
 (segment (start 133.45 92.185) (end 133.45 93.111999) (width 0.2) (layer "F.Cu") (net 6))
 (segment (start 134.999 91.159) (end 134.999 92.2) (width 0.2) (layer "F.Cu") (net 5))
 (segment (start 144.980999 94.770999) (end 144.980999 96.56934) (width 0.2) (layer "F.Cu") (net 5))
 (segment (start 136.787001 93.999) (end 135.95 93.161999) (width 0.2) (layer "F.Cu") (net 5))
 (segment (start 138.1171 94.25) (end 137.8661 93.999) (width 0.2) (layer "F.Cu") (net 5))
 (segment (start 134.7 96.374999) (end 134.7 95.6) (width 0.2) (layer "F.Cu") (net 5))
 (segment (start 144.328339 97.222) (end 135.547001 97.222) (width 0.2) (layer "F.Cu") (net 5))
 (segment (start 144.980999 96.56934) (end 144.328339 97.222) (width 0.2) (layer "F.Cu") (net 5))
 (segment (start 135.95 91.208) (end 135.901 91.159) (width 0.2) (layer "F.Cu") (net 5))
 (segment (start 135.547001 97.222) (end 134.7 96.374999) (width 0.2) (layer "F.Cu") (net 5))
 (segment (start 135.95 93.161999) (end 135.95 92.185) (width 0.2) (layer "F.Cu") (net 5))
 (segment (start 144.41 94.2) (end 144.980999 94.770999) (width 0.2) (layer "F.Cu") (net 5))
 (segment (start 139.7625 94.25) (end 138.1171 94.25) (width 0.2) (layer "F.Cu") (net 5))
 (segment (start 135.95 92.185) (end 135.95 91.208) (width 0.2) (layer "F.Cu") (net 5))
 (segment (start 137.8661 93.999) (end 136.787001 93.999) (width 0.2) (layer "F.Cu") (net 5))
 (segment (start 135.901 91.159) (end 134.999 91.159) (width 0.2) (layer "F.Cu") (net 5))
 (segment (start 143.788999 96.821) (end 136.146001 96.821) (width 0.2) (layer "F.Cu") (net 4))
 (segment (start 134.499 93.211) (end 135.401 93.211) (width 0.2) (layer "F.Cu") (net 4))
 (segment (start 136.59 94.4) (end 137.7 94.4) (width 0.2) (layer "F.Cu") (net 4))
 (segment (start 135.45 93.162) (end 135.45 92.185) (width 0.2) (layer "F.Cu") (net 4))
 (segment (start 137.7 94.4) (end 138.01645 94.71645) (width 0.2) (layer "F.Cu") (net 4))
 (segment (start 135.401 93.211) (end 136.59 94.4) (width 0.2) (layer "F.Cu") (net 4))
 (segment (start 139.100001 96.15) (end 139.7625 96.15) (width 0.2) (layer "F.Cu") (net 4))
 (segment (start 144.409999 96.2) (end 143.788999 96.821) (width 0.2) (layer "F.Cu") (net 4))
 (segment (start 136.146001 96.821) (end 135.7 96.374999) (width 0.2) (layer "F.Cu") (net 4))
 (segment (start 134.45 93.162) (end 134.499 93.211) (width 0.2) (layer "F.Cu") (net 4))
 (segment (start 135.401 93.211) (end 135.45 93.162) (width 0.2) (layer "F.Cu") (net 4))
 (segment (start 138.01645 95.066449) (end 139.100001 96.15) (width 0.2) (layer "F.Cu") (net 4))
 (segment (start 134.45 92.185) (end 134.45 93.162) (width 0.2) (layer "F.Cu") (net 4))
 (segment (start 135.7 96.374999) (end 135.7 95.6) (width 0.2) (layer "F.Cu") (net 4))
 (segment (start 138.01645 94.71645) (end 138.01645 95.066449) (width 0.2) (layer "F.Cu") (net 4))
 (segment (start 143.39 94.2) (end 142.0875 94.2) (width 0.2) (layer "F.Cu") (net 7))
 (segment (start 142.0875 94.2) (end 142.0375 94.25) (width 0.2) (layer "F.Cu") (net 7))
 (segment (start 143.390001 96.2) (end 142.0875 96.2) (width 0.2) (layer "F.Cu") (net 8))
 (segment (start 142.0875 96.2) (end 142.0375 96.15) (width 0.2) (layer "F.Cu") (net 8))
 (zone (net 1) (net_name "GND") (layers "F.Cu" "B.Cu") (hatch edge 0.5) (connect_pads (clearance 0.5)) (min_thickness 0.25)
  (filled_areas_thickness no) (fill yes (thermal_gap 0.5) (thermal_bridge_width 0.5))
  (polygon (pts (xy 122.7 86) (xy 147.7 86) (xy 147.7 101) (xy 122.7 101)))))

